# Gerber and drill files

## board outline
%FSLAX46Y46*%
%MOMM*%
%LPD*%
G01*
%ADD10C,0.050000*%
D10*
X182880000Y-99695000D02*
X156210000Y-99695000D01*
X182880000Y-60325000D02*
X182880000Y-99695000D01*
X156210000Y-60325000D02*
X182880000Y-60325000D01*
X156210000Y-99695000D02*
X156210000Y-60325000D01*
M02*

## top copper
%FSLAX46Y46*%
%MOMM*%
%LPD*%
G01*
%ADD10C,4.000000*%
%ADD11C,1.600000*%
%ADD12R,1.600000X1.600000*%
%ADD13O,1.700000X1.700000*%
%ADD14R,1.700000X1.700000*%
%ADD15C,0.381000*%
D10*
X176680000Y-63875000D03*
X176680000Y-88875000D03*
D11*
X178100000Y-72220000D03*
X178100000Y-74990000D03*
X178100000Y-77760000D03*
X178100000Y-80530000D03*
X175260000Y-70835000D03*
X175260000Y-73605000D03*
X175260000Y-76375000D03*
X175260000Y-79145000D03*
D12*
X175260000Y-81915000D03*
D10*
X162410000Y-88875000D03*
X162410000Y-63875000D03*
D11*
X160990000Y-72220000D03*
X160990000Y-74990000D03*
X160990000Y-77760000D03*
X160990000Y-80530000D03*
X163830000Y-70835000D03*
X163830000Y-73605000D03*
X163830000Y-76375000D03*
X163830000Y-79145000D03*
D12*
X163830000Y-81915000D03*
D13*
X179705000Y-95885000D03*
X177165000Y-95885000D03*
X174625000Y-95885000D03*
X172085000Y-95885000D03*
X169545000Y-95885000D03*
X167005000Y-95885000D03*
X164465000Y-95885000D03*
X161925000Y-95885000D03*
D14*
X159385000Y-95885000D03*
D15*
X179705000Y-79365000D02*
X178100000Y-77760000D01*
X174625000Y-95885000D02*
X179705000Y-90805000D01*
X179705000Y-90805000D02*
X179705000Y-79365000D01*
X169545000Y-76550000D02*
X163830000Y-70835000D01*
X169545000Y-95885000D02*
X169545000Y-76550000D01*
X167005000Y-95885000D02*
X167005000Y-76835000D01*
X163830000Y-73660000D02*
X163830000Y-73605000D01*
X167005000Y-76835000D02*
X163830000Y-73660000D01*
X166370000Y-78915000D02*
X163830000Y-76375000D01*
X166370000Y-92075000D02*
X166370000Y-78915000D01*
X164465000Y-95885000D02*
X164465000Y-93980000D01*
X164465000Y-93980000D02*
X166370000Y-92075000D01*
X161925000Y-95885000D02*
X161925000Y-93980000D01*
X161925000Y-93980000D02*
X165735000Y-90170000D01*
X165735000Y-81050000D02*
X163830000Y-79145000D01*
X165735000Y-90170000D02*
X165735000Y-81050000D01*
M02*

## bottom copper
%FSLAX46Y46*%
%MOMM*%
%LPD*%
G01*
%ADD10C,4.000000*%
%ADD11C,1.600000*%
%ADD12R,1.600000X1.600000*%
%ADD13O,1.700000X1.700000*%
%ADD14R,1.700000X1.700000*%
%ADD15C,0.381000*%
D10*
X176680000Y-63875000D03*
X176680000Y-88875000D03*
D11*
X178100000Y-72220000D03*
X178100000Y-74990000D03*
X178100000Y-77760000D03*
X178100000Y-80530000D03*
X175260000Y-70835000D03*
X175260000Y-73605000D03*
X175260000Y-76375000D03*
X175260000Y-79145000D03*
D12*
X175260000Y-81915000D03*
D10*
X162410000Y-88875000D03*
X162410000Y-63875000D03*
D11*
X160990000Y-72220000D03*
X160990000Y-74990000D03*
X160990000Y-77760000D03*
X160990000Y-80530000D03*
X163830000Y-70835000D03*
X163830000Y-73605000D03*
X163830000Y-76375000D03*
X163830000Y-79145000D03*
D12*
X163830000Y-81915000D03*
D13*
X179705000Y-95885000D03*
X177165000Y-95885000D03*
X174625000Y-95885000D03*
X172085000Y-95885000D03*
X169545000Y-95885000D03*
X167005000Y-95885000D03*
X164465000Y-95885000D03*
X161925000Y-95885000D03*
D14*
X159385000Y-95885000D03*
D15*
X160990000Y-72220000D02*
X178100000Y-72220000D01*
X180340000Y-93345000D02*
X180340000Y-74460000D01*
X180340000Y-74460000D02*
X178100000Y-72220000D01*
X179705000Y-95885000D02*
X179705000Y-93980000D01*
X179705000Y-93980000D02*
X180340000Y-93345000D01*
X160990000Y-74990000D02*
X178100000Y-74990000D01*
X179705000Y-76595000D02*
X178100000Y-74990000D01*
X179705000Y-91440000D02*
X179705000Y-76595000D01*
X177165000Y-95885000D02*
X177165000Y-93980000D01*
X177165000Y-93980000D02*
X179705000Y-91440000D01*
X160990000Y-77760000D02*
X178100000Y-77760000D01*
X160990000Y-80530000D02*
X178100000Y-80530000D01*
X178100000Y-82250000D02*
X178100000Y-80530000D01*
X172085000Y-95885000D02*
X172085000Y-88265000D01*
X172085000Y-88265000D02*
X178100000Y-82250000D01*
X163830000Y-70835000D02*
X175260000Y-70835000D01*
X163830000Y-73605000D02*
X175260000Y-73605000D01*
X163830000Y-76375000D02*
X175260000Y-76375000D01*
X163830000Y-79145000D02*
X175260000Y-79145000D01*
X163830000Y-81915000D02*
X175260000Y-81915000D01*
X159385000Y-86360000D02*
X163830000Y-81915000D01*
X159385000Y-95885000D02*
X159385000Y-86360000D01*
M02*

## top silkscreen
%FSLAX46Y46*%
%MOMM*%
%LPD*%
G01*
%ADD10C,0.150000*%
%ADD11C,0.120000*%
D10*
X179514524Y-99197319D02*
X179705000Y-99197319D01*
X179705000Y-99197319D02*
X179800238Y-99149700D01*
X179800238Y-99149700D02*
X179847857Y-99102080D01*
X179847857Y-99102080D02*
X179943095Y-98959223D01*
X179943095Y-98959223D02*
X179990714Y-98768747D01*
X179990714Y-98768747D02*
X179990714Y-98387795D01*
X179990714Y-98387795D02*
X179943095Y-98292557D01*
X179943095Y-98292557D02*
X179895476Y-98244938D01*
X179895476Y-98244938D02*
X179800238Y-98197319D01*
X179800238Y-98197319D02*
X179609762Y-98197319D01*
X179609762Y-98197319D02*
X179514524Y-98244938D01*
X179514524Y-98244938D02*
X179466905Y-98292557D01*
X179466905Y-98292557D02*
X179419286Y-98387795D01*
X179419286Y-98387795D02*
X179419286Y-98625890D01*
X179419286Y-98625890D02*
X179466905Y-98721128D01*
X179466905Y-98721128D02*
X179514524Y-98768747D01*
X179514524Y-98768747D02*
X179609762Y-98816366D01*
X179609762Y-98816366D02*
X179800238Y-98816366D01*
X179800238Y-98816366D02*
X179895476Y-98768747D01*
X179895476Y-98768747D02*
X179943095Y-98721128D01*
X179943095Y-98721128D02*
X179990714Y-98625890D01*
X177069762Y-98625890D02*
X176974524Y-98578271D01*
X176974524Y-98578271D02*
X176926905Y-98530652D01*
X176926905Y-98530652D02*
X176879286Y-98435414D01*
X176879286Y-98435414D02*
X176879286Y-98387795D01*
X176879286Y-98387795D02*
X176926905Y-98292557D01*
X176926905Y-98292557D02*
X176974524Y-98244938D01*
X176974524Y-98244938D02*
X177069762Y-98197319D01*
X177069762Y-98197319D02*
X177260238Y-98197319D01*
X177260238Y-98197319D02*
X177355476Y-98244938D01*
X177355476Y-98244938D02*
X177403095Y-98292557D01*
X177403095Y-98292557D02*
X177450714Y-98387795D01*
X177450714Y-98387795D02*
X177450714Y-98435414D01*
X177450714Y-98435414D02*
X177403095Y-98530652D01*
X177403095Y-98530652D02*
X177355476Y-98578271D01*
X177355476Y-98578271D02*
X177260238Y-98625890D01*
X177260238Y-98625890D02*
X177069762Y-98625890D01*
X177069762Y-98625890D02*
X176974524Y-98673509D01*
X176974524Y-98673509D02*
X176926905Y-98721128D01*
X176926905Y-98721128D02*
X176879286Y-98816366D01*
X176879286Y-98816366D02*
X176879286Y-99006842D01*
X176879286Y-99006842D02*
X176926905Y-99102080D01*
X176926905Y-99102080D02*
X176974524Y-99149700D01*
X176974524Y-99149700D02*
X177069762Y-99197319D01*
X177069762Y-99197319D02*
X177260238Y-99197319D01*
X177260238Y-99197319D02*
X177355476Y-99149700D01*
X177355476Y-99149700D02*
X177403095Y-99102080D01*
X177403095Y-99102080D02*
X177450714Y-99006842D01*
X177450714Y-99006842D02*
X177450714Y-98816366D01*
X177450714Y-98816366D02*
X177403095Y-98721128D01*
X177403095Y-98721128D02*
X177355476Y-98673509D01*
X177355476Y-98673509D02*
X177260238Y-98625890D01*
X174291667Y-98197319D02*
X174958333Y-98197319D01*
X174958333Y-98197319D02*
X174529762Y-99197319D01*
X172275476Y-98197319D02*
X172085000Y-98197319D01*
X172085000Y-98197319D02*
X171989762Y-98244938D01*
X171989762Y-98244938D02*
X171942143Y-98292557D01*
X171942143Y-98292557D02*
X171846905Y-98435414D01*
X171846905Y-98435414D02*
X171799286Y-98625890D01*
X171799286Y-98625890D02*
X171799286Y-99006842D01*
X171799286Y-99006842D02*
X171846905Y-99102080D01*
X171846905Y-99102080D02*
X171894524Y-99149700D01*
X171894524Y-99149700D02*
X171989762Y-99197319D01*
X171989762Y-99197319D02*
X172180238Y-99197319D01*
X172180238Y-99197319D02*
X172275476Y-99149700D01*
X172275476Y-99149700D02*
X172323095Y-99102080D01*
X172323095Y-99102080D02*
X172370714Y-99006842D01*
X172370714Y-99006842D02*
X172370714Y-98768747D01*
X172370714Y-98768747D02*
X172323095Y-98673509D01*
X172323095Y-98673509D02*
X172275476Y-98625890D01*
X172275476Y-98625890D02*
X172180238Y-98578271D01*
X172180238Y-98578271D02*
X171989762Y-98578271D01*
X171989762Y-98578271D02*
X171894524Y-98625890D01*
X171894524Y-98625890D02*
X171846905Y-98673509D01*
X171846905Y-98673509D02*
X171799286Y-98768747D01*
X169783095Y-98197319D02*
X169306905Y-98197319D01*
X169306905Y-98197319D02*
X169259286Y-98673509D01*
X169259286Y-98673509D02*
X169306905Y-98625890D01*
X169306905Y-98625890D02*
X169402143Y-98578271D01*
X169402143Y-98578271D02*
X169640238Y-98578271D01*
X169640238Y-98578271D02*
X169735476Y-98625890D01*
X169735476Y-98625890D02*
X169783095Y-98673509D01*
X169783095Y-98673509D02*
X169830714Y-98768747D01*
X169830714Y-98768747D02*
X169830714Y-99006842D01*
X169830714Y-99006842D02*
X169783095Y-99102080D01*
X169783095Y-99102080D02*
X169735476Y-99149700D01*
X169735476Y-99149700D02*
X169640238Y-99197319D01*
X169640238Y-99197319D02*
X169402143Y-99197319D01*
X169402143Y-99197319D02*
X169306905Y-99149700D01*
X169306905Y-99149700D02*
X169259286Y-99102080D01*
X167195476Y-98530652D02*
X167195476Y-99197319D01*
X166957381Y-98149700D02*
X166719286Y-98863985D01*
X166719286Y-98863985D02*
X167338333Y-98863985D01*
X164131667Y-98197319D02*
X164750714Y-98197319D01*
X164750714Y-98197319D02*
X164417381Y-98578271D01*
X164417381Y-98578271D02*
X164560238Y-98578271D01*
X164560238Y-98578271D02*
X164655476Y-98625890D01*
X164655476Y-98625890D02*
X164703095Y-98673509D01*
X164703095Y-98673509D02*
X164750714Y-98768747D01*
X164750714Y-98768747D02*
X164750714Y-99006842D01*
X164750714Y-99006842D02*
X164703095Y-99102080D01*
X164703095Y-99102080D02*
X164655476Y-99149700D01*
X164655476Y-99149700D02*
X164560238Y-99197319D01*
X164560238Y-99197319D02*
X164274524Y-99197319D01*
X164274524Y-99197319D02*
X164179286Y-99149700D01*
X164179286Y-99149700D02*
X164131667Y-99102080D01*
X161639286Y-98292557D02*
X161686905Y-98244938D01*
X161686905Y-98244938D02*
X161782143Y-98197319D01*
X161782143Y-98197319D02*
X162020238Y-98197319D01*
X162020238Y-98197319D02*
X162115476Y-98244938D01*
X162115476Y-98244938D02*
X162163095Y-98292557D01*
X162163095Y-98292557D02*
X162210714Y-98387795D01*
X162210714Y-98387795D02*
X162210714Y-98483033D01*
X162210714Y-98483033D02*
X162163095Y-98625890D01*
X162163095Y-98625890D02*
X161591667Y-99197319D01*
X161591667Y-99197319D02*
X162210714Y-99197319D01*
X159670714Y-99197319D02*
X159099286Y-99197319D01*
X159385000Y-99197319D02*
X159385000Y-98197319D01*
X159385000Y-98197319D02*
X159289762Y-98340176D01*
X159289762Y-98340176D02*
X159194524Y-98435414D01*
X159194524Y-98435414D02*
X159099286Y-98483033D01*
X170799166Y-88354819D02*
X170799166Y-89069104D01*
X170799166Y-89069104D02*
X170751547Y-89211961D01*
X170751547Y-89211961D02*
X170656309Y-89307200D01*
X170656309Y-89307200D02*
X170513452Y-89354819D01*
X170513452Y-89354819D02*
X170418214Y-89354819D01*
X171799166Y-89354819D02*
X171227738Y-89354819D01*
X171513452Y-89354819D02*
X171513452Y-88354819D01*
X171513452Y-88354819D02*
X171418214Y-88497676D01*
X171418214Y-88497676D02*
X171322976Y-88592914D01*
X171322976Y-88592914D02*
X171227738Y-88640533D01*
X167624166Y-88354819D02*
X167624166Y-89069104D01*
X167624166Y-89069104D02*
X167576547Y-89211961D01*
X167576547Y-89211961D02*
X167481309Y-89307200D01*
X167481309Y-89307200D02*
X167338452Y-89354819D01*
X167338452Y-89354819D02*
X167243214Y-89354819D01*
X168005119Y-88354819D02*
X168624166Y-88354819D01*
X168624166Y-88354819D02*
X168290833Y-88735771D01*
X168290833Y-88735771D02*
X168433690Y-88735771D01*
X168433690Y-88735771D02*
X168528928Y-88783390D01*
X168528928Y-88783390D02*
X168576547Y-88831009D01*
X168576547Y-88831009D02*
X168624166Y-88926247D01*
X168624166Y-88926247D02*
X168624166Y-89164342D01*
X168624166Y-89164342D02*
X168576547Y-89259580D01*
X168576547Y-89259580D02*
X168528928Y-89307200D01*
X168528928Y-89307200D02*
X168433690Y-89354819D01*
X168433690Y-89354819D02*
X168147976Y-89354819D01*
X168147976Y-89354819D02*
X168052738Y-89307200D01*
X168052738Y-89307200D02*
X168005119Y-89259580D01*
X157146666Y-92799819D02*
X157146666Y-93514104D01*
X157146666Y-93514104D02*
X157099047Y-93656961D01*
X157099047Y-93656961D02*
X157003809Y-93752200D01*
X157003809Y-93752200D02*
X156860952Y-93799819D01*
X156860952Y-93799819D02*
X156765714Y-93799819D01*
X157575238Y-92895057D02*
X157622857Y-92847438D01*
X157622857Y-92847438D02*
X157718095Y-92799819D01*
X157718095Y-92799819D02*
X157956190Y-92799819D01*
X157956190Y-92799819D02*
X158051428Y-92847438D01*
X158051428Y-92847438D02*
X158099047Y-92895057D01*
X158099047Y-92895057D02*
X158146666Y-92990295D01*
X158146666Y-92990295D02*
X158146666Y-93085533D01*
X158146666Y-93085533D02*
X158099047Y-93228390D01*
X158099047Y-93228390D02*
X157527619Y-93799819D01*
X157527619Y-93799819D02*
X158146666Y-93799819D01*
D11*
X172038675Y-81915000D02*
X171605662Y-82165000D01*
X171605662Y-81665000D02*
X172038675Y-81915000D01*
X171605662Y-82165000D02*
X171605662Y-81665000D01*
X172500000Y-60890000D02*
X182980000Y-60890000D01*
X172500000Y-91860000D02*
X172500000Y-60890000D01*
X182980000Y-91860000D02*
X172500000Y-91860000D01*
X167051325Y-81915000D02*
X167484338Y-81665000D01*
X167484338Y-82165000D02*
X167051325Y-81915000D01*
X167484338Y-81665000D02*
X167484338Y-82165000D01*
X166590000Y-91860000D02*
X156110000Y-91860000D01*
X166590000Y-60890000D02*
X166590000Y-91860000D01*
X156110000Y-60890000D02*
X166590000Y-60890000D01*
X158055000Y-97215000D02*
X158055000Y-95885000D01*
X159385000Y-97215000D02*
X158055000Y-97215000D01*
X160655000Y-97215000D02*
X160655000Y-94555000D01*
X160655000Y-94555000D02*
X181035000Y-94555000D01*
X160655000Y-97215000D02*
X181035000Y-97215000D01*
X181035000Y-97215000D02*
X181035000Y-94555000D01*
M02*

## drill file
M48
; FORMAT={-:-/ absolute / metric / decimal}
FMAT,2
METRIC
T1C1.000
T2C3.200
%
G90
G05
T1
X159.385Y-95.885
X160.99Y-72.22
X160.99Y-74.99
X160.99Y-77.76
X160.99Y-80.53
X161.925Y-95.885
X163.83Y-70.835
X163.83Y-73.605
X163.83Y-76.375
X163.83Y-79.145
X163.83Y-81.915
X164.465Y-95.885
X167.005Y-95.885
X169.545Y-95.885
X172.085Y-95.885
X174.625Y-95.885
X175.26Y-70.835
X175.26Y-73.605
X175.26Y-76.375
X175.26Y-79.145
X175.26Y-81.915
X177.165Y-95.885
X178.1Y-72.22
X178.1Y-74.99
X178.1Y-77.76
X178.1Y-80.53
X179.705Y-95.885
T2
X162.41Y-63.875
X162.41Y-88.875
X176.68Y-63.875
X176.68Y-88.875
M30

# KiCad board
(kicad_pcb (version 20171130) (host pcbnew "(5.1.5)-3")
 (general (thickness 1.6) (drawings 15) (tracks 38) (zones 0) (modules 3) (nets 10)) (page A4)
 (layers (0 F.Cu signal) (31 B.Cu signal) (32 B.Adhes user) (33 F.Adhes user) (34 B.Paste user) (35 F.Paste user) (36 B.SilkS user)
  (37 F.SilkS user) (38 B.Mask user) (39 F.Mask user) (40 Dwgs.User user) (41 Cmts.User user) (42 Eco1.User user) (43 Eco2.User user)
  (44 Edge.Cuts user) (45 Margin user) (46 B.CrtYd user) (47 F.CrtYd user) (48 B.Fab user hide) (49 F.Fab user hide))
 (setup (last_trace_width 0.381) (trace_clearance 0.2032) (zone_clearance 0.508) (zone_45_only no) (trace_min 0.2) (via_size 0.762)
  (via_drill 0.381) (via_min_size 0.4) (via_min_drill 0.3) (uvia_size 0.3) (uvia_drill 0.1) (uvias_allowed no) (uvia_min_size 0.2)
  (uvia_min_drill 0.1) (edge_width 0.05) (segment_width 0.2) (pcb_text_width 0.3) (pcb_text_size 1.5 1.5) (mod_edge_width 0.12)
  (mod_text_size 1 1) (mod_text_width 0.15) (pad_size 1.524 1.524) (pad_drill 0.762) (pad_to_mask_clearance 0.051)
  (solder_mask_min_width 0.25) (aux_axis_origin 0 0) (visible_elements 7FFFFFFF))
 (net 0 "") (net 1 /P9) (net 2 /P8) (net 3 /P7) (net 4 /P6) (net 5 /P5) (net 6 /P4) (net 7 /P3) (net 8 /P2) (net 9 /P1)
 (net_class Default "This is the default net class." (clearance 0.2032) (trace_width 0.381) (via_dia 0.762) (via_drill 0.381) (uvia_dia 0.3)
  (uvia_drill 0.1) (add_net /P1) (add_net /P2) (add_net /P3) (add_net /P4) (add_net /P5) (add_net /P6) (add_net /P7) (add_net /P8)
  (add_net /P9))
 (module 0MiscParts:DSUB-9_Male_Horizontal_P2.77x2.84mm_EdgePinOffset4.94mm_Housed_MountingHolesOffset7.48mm (layer F.Cu)
  (at 175.26 81.915 90)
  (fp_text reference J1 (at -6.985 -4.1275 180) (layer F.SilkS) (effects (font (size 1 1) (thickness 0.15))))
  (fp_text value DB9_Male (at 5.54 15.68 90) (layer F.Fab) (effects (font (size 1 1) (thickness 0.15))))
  (fp_line (start 0 -3.221325) (end -0.25 -3.654338) (layer F.SilkS) (width 0.12))
  (fp_line (start 0.25 -3.654338) (end 0 -3.221325) (layer F.SilkS) (width 0.12))
  (fp_line (start -0.25 -3.654338) (end 0.25 -3.654338) (layer F.SilkS) (width 0.12))
  (fp_line (start 21.025 -2.76) (end 21.025 7.72) (layer F.SilkS) (width 0.12))
  (fp_line (start -9.945 -2.76) (end 21.025 -2.76) (layer F.SilkS) (width 0.12))
  (fp_line (start -9.945 7.72) (end -9.945 -2.76) (layer F.SilkS) (width 0.12))
  (pad 0 thru_hole circle (at 18.04 1.42 90) (size 4 4) (drill 3.2) (layers *.Cu *.Mask))
  (pad 0 thru_hole circle (at -6.96 1.42 90) (size 4 4) (drill 3.2) (layers *.Cu *.Mask))
  (pad 9 thru_hole circle (at 9.695 2.84 90) (size 1.6 1.6) (drill 1) (layers *.Cu *.Mask) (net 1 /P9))
  (pad 8 thru_hole circle (at 6.925 2.84 90) (size 1.6 1.6) (drill 1) (layers *.Cu *.Mask) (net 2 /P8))
  (pad 7 thru_hole circle (at 4.155 2.84 90) (size 1.6 1.6) (drill 1) (layers *.Cu *.Mask) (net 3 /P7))
  (pad 6 thru_hole circle (at 1.385 2.84 90) (size 1.6 1.6) (drill 1) (layers *.Cu *.Mask) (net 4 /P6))
  (pad 5 thru_hole circle (at 11.08 0 90) (size 1.6 1.6) (drill 1) (layers *.Cu *.Mask) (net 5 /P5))
  (pad 4 thru_hole circle (at 8.31 0 90) (size 1.6 1.6) (drill 1) (layers *.Cu *.Mask) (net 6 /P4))
  (pad 3 thru_hole circle (at 5.54 0 90) (size 1.6 1.6) (drill 1) (layers *.Cu *.Mask) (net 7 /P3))
  (pad 2 thru_hole circle (at 2.77 0 90) (size 1.6 1.6) (drill 1) (layers *.Cu *.Mask) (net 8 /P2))
  (pad 1 thru_hole rect (at 0 0 90) (size 1.6 1.6) (drill 1) (layers *.Cu *.Mask) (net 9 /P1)))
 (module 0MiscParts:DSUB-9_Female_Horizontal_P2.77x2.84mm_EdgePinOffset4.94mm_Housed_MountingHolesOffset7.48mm (layer F.Cu)
  (at 163.83 81.915 270)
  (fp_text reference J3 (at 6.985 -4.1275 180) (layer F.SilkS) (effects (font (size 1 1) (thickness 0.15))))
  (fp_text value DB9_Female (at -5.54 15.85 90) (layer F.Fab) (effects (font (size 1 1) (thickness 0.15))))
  (fp_line (start 0 -3.221325) (end -0.25 -3.654338) (layer F.SilkS) (width 0.12))
  (fp_line (start 0.25 -3.654338) (end 0 -3.221325) (layer F.SilkS) (width 0.12))
  (fp_line (start -0.25 -3.654338) (end 0.25 -3.654338) (layer F.SilkS) (width 0.12))
  (fp_line (start 9.945 -2.76) (end 9.945 7.72) (layer F.SilkS) (width 0.12))
  (fp_line (start -21.025 -2.76) (end 9.945 -2.76) (layer F.SilkS) (width 0.12))
  (fp_line (start -21.025 7.72) (end -21.025 -2.76) (layer F.SilkS) (width 0.12))
  (pad 0 thru_hole circle (at 6.96 1.42 270) (size 4 4) (drill 3.2) (layers *.Cu *.Mask))
  (pad 0 thru_hole circle (at -18.04 1.42 270) (size 4 4) (drill 3.2) (layers *.Cu *.Mask))
  (pad 9 thru_hole circle (at -9.695 2.84 270) (size 1.6 1.6) (drill 1) (layers *.Cu *.Mask) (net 1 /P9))
  (pad 8 thru_hole circle (at -6.925 2.84 270) (size 1.6 1.6) (drill 1) (layers *.Cu *.Mask) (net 2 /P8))
  (pad 7 thru_hole circle (at -4.155 2.84 270) (size 1.6 1.6) (drill 1) (layers *.Cu *.Mask) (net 3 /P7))
  (pad 6 thru_hole circle (at -1.385 2.84 270) (size 1.6 1.6) (drill 1) (layers *.Cu *.Mask) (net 4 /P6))
  (pad 5 thru_hole circle (at -11.08 0 270) (size 1.6 1.6) (drill 1) (layers *.Cu *.Mask) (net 5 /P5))
  (pad 4 thru_hole circle (at -8.31 0 270) (size 1.6 1.6) (drill 1) (layers *.Cu *.Mask) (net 6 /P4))
  (pad 3 thru_hole circle (at -5.54 0 270) (size 1.6 1.6) (drill 1) (layers *.Cu *.Mask) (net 7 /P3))
  (pad 2 thru_hole circle (at -2.77 0 270) (size 1.6 1.6) (drill 1) (layers *.Cu *.Mask) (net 8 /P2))
  (pad 1 thru_hole rect (at 0 0 270) (size 1.6 1.6) (drill 1) (layers *.Cu *.Mask) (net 9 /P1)))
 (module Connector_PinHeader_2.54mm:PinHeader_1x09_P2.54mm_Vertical (layer F.Cu) (at 159.385 95.885 90)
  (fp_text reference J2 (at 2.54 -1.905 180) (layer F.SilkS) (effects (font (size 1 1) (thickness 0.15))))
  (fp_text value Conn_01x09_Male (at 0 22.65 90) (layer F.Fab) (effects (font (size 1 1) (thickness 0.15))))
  (fp_line (start -1.33 -1.33) (end 0 -1.33) (layer F.SilkS) (width 0.12))
  (fp_line (start -1.33 0) (end -1.33 -1.33) (layer F.SilkS) (width 0.12))
  (fp_line (start -1.33 1.27) (end 1.33 1.27) (layer F.SilkS) (width 0.12))
  (fp_line (start 1.33 1.27) (end 1.33 21.65) (layer F.SilkS) (width 0.12))
  (fp_line (start -1.33 1.27) (end -1.33 21.65) (layer F.SilkS) (width 0.12))
  (fp_line (start -1.33 21.65) (end 1.33 21.65) (layer F.SilkS) (width 0.12))
  (pad 9 thru_hole oval (at 0 20.32 90) (size 1.7 1.7) (drill 1) (layers *.Cu *.Mask) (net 1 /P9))
  (pad 8 thru_hole oval (at 0 17.78 90) (size 1.7 1.7) (drill 1) (layers *.Cu *.Mask) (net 2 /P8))
  (pad 7 thru_hole oval (at 0 15.24 90) (size 1.7 1.7) (drill 1) (layers *.Cu *.Mask) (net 3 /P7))
  (pad 6 thru_hole oval (at 0 12.7 90) (size 1.7 1.7) (drill 1) (layers *.Cu *.Mask) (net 4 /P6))
  (pad 5 thru_hole oval (at 0 10.16 90) (size 1.7 1.7) (drill 1) (layers *.Cu *.Mask) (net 5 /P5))
  (pad 4 thru_hole oval (at 0 7.62 90) (size 1.7 1.7) (drill 1) (layers *.Cu *.Mask) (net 6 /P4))
  (pad 3 thru_hole oval (at 0 5.08 90) (size 1.7 1.7) (drill 1) (layers *.Cu *.Mask) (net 7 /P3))
  (pad 2 thru_hole oval (at 0 2.54 90) (size 1.7 1.7) (drill 1) (layers *.Cu *.Mask) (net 8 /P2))
  (pad 1 thru_hole rect (at 0 0 90) (size 1.7 1.7) (drill 1) (layers *.Cu *.Mask) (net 9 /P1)))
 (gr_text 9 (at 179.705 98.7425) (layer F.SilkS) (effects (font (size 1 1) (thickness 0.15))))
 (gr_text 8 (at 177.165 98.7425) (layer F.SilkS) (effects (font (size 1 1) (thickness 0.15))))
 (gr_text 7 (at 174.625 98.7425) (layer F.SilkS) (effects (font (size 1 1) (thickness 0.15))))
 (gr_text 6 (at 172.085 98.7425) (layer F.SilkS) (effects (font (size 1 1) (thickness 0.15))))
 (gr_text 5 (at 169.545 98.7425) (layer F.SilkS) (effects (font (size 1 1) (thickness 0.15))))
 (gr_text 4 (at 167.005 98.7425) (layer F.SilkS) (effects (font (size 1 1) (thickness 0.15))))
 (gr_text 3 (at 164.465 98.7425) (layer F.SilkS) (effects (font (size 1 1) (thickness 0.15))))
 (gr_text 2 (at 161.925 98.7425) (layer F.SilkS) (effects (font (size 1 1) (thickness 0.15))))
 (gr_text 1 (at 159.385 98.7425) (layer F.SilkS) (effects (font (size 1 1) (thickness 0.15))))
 (gr_line (start 182.88 99.695) (end 156.21 99.695) (layer Edge.Cuts) (width 0.05))
 (gr_line (start 182.88 60.325) (end 182.88 99.695) (layer Edge.Cuts) (width 0.05))
 (gr_line (start 156.21 60.325) (end 182.88 60.325) (layer Edge.Cuts) (width 0.05))
 (gr_line (start 156.21 99.695) (end 156.21 60.325) (layer Edge.Cuts) (width 0.05))
 (segment (start 160.99 72.22) (end 178.1 72.22) (width 0.381) (layer B.Cu) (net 1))
 (segment (start 180.34 93.345) (end 180.34 74.46) (width 0.381) (layer B.Cu) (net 1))
 (segment (start 180.34 74.46) (end 178.1 72.22) (width 0.381) (layer B.Cu) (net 1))
 (segment (start 179.705 95.885) (end 179.705 93.98) (width 0.381) (layer B.Cu) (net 1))
 (segment (start 179.705 93.98) (end 180.34 93.345) (width 0.381) (layer B.Cu) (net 1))
 (segment (start 160.99 74.99) (end 178.1 74.99) (width 0.381) (layer B.Cu) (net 2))
 (segment (start 179.705 76.595) (end 178.1 74.99) (width 0.381) (layer B.Cu) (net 2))
 (segment (start 179.705 91.44) (end 179.705 76.595) (width 0.381) (layer B.Cu) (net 2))
 (segment (start 177.165 95.885) (end 177.165 93.98) (width 0.381) (layer B.Cu) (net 2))
 (segment (start 177.165 93.98) (end 179.705 91.44) (width 0.381) (layer B.Cu) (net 2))
 (segment (start 160.99 77.76) (end 178.1 77.76) (width 0.381) (layer B.Cu) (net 3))
 (segment (start 179.705 79.365) (end 178.1 77.76) (width 0.381) (layer F.Cu) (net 3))
 (segment (start 174.625 95.885) (end 179.705 90.805) (width 0.381) (layer F.Cu) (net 3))
 (segment (start 179.705 90.805) (end 179.705 79.365) (width 0.381) (layer F.Cu) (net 3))
 (segment (start 160.99 80.53) (end 178.1 80.53) (width 0.381) (layer B.Cu) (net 4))
 (segment (start 178.1 82.25) (end 178.1 80.53) (width 0.381) (layer B.Cu) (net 4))
 (segment (start 172.085 95.885) (end 172.085 88.265) (width 0.381) (layer B.Cu) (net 4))
 (segment (start 172.085 88.265) (end 178.1 82.25) (width 0.381) (layer B.Cu) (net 4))
 (segment (start 163.83 70.835) (end 175.26 70.835) (width 0.381) (layer B.Cu) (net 5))
 (segment (start 169.545 76.55) (end 163.83 70.835) (width 0.381) (layer F.Cu) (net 5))
 (segment (start 169.545 95.885) (end 169.545 76.55) (width 0.381) (layer F.Cu) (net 5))
 (segment (start 163.83 73.605) (end 175.26 73.605) (width 0.381) (layer B.Cu) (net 6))
 (segment (start 167.005 95.885) (end 167.005 76.835) (width 0.381) (layer F.Cu) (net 6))
 (segment (start 163.83 73.66) (end 163.83 73.605) (width 0.381) (layer F.Cu) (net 6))
 (segment (start 167.005 76.835) (end 163.83 73.66) (width 0.381) (layer F.Cu) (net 6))
 (segment (start 163.83 76.375) (end 175.26 76.375) (width 0.381) (layer B.Cu) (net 7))
 (segment (start 166.37 78.915) (end 163.83 76.375) (width 0.381) (layer F.Cu) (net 7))
 (segment (start 166.37 92.075) (end 166.37 78.915) (width 0.381) (layer F.Cu) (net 7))
 (segment (start 164.465 95.885) (end 164.465 93.98) (width 0.381) (layer F.Cu) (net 7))
 (segment (start 164.465 93.98) (end 166.37 92.075) (width 0.381) (layer F.Cu) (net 7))
 (segment (start 163.83 79.145) (end 175.26 79.145) (width 0.381) (layer B.Cu) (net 8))
 (segment (start 161.925 95.885) (end 161.925 93.98) (width 0.381) (layer F.Cu) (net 8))
 (segment (start 161.925 93.98) (end 165.735 90.17) (width 0.381) (layer F.Cu) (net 8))
 (segment (start 165.735 81.05) (end 163.83 79.145) (width 0.381) (layer F.Cu) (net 8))
 (segment (start 165.735 90.17) (end 165.735 81.05) (width 0.381) (layer F.Cu) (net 8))
 (segment (start 163.83 81.915) (end 175.26 81.915) (width 0.381) (layer B.Cu) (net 9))
 (segment (start 159.385 86.36) (end 163.83 81.915) (width 0.381) (layer B.Cu) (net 9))
 (segment (start 159.385 95.885) (end 159.385 86.36) (width 0.381) (layer B.Cu) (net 9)))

